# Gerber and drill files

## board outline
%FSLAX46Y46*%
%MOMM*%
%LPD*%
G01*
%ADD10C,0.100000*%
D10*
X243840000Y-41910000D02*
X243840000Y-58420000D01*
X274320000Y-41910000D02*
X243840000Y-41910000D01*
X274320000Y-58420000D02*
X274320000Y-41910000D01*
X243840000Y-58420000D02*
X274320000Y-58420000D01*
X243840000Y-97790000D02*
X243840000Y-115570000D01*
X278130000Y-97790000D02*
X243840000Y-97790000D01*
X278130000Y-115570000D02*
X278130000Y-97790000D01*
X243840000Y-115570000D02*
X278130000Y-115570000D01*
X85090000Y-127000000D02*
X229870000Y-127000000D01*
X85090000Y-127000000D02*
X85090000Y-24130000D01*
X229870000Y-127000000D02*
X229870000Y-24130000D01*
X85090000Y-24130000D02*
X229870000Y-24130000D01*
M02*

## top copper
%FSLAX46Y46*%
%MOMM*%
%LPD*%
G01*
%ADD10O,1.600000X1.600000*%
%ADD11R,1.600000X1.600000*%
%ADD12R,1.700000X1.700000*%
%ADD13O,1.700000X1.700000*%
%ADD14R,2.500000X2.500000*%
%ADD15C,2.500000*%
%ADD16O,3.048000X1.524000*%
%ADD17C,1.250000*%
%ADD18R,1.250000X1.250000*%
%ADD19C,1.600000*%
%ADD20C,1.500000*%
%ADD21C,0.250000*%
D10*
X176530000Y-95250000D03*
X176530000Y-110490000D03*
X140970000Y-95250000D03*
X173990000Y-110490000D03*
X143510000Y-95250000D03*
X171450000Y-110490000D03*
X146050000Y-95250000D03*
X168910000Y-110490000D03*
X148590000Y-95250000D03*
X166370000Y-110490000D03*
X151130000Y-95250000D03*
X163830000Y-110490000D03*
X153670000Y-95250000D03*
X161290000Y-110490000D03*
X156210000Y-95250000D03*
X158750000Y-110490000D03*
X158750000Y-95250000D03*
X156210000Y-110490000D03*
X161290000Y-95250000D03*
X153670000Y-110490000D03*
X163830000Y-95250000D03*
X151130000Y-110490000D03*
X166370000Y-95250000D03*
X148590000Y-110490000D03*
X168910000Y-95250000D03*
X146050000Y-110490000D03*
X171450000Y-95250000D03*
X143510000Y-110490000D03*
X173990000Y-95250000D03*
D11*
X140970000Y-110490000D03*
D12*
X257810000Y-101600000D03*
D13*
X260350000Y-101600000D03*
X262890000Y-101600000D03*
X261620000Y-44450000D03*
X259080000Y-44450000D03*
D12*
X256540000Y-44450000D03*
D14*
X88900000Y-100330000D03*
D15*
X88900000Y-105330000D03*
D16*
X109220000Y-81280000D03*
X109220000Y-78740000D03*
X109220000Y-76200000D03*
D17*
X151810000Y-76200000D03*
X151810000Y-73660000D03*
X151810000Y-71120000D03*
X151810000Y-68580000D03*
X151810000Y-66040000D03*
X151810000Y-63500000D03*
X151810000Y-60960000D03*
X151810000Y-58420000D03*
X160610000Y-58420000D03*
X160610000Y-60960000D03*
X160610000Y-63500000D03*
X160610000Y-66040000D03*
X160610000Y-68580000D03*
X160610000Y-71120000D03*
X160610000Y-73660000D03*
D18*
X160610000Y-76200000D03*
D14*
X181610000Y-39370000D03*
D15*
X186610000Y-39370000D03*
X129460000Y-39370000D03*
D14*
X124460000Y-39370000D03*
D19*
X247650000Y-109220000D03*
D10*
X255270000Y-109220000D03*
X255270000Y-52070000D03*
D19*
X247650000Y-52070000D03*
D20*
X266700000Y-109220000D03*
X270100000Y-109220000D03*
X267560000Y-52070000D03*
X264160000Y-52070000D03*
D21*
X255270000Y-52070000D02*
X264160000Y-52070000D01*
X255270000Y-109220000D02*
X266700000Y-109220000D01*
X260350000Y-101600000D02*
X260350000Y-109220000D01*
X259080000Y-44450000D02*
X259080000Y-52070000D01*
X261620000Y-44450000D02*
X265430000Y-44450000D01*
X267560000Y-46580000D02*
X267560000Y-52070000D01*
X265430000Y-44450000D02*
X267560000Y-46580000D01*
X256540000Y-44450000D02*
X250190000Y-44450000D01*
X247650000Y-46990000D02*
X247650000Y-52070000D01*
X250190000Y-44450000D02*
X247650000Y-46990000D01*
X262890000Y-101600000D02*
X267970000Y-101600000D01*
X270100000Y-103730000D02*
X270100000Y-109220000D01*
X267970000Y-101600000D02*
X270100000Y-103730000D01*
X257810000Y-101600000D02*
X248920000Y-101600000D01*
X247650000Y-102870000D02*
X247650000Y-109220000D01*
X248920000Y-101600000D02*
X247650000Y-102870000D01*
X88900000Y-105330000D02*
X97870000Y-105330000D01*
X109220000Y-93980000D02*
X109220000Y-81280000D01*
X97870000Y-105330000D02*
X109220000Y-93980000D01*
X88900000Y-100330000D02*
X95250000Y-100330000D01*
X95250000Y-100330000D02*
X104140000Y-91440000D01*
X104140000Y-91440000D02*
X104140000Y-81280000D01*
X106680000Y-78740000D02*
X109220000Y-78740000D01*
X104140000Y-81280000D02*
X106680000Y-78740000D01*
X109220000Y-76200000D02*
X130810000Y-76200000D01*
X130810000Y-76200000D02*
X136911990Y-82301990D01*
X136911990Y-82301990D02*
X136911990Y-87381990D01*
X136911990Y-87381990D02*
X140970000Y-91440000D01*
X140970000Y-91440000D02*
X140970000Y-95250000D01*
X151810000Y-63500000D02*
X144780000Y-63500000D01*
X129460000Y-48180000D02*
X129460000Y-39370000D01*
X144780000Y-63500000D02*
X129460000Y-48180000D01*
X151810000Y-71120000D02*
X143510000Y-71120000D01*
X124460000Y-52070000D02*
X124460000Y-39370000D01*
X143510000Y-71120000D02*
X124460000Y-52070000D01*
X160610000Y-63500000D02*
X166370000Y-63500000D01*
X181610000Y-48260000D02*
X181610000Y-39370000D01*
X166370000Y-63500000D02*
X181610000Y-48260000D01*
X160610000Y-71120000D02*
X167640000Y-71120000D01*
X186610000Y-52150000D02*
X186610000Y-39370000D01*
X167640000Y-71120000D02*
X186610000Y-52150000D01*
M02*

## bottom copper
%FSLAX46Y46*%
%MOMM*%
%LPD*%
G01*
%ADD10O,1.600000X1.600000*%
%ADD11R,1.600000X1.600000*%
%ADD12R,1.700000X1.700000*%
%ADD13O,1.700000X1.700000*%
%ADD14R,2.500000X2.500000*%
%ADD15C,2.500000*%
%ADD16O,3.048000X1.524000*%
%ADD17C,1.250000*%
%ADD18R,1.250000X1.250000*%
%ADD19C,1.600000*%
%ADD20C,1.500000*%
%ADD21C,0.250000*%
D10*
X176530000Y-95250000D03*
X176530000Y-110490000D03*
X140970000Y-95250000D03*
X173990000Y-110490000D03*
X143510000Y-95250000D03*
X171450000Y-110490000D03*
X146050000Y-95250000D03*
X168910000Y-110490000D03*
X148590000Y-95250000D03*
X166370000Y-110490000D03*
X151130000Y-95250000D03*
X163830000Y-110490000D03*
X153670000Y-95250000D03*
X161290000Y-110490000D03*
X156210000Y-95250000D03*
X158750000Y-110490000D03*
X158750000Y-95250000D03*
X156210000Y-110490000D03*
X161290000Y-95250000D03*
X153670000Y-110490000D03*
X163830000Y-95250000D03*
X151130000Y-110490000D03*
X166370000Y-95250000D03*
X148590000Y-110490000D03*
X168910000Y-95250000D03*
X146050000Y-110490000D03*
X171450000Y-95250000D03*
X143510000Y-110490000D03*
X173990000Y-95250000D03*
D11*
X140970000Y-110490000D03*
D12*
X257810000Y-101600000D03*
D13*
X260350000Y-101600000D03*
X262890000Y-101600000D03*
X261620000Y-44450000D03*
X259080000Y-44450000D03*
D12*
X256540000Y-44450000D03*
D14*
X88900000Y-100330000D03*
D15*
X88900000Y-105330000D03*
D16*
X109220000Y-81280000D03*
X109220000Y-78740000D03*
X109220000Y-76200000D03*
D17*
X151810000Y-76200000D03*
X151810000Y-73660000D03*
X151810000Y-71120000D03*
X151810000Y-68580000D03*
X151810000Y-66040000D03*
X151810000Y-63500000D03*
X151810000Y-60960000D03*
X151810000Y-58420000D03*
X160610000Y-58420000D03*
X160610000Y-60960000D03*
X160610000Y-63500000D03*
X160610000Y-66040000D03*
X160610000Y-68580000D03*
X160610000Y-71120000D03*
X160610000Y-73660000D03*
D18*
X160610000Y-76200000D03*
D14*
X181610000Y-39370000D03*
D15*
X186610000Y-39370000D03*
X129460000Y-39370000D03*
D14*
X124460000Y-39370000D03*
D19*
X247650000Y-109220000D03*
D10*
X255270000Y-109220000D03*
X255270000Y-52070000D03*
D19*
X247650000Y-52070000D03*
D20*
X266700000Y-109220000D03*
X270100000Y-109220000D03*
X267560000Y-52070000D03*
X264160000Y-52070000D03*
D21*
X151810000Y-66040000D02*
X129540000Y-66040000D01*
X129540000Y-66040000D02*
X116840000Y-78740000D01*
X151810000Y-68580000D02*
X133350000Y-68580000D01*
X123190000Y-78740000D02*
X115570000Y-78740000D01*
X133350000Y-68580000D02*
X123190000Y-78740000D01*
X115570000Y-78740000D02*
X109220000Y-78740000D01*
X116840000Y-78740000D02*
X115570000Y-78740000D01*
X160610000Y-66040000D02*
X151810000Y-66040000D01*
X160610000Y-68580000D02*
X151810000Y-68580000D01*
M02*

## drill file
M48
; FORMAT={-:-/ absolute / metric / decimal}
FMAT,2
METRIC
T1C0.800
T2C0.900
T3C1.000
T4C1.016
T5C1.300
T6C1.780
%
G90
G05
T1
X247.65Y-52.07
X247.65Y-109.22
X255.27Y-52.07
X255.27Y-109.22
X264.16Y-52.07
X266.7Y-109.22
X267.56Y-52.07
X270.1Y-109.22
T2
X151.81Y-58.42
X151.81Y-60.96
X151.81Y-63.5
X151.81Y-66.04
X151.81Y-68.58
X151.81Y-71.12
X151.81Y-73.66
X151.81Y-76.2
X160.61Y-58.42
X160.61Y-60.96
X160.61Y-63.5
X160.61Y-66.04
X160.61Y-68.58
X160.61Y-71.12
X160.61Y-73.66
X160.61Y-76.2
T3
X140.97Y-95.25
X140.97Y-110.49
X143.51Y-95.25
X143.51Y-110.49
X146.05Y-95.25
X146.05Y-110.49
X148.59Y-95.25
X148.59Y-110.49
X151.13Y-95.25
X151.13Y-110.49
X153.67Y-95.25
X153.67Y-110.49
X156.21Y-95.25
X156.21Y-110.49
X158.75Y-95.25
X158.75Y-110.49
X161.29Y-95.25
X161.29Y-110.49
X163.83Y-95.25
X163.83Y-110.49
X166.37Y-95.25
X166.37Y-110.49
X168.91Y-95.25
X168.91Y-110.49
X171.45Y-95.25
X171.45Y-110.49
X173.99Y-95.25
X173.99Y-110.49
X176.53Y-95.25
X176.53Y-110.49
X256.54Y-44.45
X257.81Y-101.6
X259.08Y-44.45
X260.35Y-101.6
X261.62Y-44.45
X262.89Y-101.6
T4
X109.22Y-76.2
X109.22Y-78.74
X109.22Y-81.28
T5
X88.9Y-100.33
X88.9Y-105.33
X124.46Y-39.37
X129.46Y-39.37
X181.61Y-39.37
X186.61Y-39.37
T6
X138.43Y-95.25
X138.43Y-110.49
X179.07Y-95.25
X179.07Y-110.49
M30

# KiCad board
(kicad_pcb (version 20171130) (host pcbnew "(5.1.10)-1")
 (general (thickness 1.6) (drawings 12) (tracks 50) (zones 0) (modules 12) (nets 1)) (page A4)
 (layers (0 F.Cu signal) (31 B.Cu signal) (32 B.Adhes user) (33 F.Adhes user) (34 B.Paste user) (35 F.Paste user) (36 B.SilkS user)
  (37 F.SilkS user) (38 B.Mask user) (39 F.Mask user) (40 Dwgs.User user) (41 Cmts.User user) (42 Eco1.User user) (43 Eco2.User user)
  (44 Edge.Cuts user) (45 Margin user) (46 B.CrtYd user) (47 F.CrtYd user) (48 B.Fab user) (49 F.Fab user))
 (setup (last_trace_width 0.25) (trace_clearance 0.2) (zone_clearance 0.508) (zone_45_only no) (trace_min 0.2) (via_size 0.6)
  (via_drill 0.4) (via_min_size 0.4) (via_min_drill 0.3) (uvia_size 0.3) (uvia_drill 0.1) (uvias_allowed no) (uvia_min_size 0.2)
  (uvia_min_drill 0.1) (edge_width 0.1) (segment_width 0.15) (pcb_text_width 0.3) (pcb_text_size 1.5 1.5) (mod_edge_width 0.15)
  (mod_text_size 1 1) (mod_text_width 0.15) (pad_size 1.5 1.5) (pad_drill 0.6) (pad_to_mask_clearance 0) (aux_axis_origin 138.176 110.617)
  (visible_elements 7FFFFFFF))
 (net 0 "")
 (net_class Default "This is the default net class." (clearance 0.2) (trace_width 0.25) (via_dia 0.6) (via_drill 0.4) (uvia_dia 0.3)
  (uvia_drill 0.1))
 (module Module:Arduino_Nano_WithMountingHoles (layer F.Cu) (at 140.97 110.49 90)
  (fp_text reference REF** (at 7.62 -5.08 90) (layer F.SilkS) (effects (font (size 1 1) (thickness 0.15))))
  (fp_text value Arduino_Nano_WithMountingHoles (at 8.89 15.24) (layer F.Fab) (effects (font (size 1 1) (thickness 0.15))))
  (pad "" np_thru_hole circle (at 0 38.1 90) (size 1.78 1.78) (drill 1.78) (layers *.Cu *.Mask))
  (pad "" np_thru_hole circle (at 15.24 38.1 90) (size 1.78 1.78) (drill 1.78) (layers *.Cu *.Mask))
  (pad "" np_thru_hole circle (at 15.24 -2.54 90) (size 1.78 1.78) (drill 1.78) (layers *.Cu *.Mask))
  (pad "" np_thru_hole circle (at 0 -2.54 90) (size 1.78 1.78) (drill 1.78) (layers *.Cu *.Mask))
  (pad 16 thru_hole oval (at 15.24 35.56 90) (size 1.6 1.6) (drill 1) (layers *.Cu *.Mask))
  (pad 15 thru_hole oval (at 0 35.56 90) (size 1.6 1.6) (drill 1) (layers *.Cu *.Mask))
  (pad 30 thru_hole oval (at 15.24 0 90) (size 1.6 1.6) (drill 1) (layers *.Cu *.Mask))
  (pad 14 thru_hole oval (at 0 33.02 90) (size 1.6 1.6) (drill 1) (layers *.Cu *.Mask))
  (pad 29 thru_hole oval (at 15.24 2.54 90) (size 1.6 1.6) (drill 1) (layers *.Cu *.Mask))
  (pad 13 thru_hole oval (at 0 30.48 90) (size 1.6 1.6) (drill 1) (layers *.Cu *.Mask))
  (pad 28 thru_hole oval (at 15.24 5.08 90) (size 1.6 1.6) (drill 1) (layers *.Cu *.Mask))
  (pad 12 thru_hole oval (at 0 27.94 90) (size 1.6 1.6) (drill 1) (layers *.Cu *.Mask))
  (pad 27 thru_hole oval (at 15.24 7.62 90) (size 1.6 1.6) (drill 1) (layers *.Cu *.Mask))
  (pad 11 thru_hole oval (at 0 25.4 90) (size 1.6 1.6) (drill 1) (layers *.Cu *.Mask))
  (pad 26 thru_hole oval (at 15.24 10.16 90) (size 1.6 1.6) (drill 1) (layers *.Cu *.Mask))
  (pad 10 thru_hole oval (at 0 22.86 90) (size 1.6 1.6) (drill 1) (layers *.Cu *.Mask))
  (pad 25 thru_hole oval (at 15.24 12.7 90) (size 1.6 1.6) (drill 1) (layers *.Cu *.Mask))
  (pad 9 thru_hole oval (at 0 20.32 90) (size 1.6 1.6) (drill 1) (layers *.Cu *.Mask))
  (pad 24 thru_hole oval (at 15.24 15.24 90) (size 1.6 1.6) (drill 1) (layers *.Cu *.Mask))
  (pad 8 thru_hole oval (at 0 17.78 90) (size 1.6 1.6) (drill 1) (layers *.Cu *.Mask))
  (pad 23 thru_hole oval (at 15.24 17.78 90) (size 1.6 1.6) (drill 1) (layers *.Cu *.Mask))
  (pad 7 thru_hole oval (at 0 15.24 90) (size 1.6 1.6) (drill 1) (layers *.Cu *.Mask))
  (pad 22 thru_hole oval (at 15.24 20.32 90) (size 1.6 1.6) (drill 1) (layers *.Cu *.Mask))
  (pad 6 thru_hole oval (at 0 12.7 90) (size 1.6 1.6) (drill 1) (layers *.Cu *.Mask))
  (pad 21 thru_hole oval (at 15.24 22.86 90) (size 1.6 1.6) (drill 1) (layers *.Cu *.Mask))
  (pad 5 thru_hole oval (at 0 10.16 90) (size 1.6 1.6) (drill 1) (layers *.Cu *.Mask))
  (pad 20 thru_hole oval (at 15.24 25.4 90) (size 1.6 1.6) (drill 1) (layers *.Cu *.Mask))
  (pad 4 thru_hole oval (at 0 7.62 90) (size 1.6 1.6) (drill 1) (layers *.Cu *.Mask))
  (pad 19 thru_hole oval (at 15.24 27.94 90) (size 1.6 1.6) (drill 1) (layers *.Cu *.Mask))
  (pad 3 thru_hole oval (at 0 5.08 90) (size 1.6 1.6) (drill 1) (layers *.Cu *.Mask))
  (pad 18 thru_hole oval (at 15.24 30.48 90) (size 1.6 1.6) (drill 1) (layers *.Cu *.Mask))
  (pad 2 thru_hole oval (at 0 2.54 90) (size 1.6 1.6) (drill 1) (layers *.Cu *.Mask))
  (pad 17 thru_hole oval (at 15.24 33.02 90) (size 1.6 1.6) (drill 1) (layers *.Cu *.Mask))
  (pad 1 thru_hole rect (at 0 0 90) (size 1.6 1.6) (drill 1) (layers *.Cu *.Mask)))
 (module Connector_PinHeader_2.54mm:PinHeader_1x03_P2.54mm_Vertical (layer F.Cu) (at 257.81 101.6 90)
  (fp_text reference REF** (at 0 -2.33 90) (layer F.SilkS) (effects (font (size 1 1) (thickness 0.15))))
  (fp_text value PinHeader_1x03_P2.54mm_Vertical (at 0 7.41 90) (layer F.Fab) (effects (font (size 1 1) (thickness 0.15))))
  (pad 1 thru_hole rect (at 0 0 90) (size 1.7 1.7) (drill 1) (layers *.Cu *.Mask))
  (pad 2 thru_hole oval (at 0 2.54 90) (size 1.7 1.7) (drill 1) (layers *.Cu *.Mask))
  (pad 3 thru_hole oval (at 0 5.08 90) (size 1.7 1.7) (drill 1) (layers *.Cu *.Mask)))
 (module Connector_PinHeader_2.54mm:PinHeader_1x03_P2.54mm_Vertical (layer F.Cu) (at 256.54 44.45 90)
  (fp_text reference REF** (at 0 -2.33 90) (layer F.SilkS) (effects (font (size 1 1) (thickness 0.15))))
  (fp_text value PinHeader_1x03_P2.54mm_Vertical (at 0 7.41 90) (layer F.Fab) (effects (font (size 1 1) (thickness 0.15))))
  (pad 3 thru_hole oval (at 0 5.08 90) (size 1.7 1.7) (drill 1) (layers *.Cu *.Mask))
  (pad 2 thru_hole oval (at 0 2.54 90) (size 1.7 1.7) (drill 1) (layers *.Cu *.Mask))
  (pad 1 thru_hole rect (at 0 0 90) (size 1.7 1.7) (drill 1) (layers *.Cu *.Mask)))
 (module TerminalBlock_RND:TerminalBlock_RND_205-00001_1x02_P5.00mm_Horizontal (layer F.Cu) (at 88.9 100.33 270)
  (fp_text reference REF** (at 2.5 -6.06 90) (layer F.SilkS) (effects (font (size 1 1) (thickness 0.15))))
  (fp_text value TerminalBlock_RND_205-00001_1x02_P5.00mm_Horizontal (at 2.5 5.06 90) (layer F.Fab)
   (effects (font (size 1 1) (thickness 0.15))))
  (pad 1 thru_hole rect (at 0 0 270) (size 2.5 2.5) (drill 1.3) (layers *.Cu *.Mask))
  (pad 2 thru_hole circle (at 5 0 270) (size 2.5 2.5) (drill 1.3) (layers *.Cu *.Mask)))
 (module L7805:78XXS (layer F.Cu) (at 111.76 78.74 270)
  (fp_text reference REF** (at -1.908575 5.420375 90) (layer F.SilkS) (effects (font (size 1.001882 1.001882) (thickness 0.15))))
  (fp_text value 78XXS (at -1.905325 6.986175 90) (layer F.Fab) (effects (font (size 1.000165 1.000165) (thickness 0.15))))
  (pad OUT thru_hole oval (at 2.54 2.54 270) (size 1.524 3.048) (drill 1.016) (layers *.Cu *.Mask))
  (pad GND thru_hole oval (at 0 2.54 270) (size 1.524 3.048) (drill 1.016) (layers *.Cu *.Mask))
  (pad IN thru_hole oval (at -2.54 2.54 270) (size 1.524 3.048) (drill 1.016) (layers *.Cu *.Mask)))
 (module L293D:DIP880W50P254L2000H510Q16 (layer F.Cu) (at 156.21 67.31 180)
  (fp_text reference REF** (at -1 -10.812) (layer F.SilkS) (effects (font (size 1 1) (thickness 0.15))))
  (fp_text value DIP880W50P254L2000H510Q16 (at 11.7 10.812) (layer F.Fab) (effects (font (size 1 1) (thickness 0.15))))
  (pad 16 thru_hole circle (at 4.4 -8.89 180) (size 1.25 1.25) (drill 0.9) (layers *.Cu *.Mask))
  (pad 15 thru_hole circle (at 4.4 -6.35 180) (size 1.25 1.25) (drill 0.9) (layers *.Cu *.Mask))
  (pad 14 thru_hole circle (at 4.4 -3.81 180) (size 1.25 1.25) (drill 0.9) (layers *.Cu *.Mask))
  (pad 13 thru_hole circle (at 4.4 -1.27 180) (size 1.25 1.25) (drill 0.9) (layers *.Cu *.Mask))
  (pad 12 thru_hole circle (at 4.4 1.27 180) (size 1.25 1.25) (drill 0.9) (layers *.Cu *.Mask))
  (pad 11 thru_hole circle (at 4.4 3.81 180) (size 1.25 1.25) (drill 0.9) (layers *.Cu *.Mask))
  (pad 10 thru_hole circle (at 4.4 6.35 180) (size 1.25 1.25) (drill 0.9) (layers *.Cu *.Mask))
  (pad 9 thru_hole circle (at 4.4 8.89 180) (size 1.25 1.25) (drill 0.9) (layers *.Cu *.Mask))
  (pad 8 thru_hole circle (at -4.4 8.89 180) (size 1.25 1.25) (drill 0.9) (layers *.Cu *.Mask))
  (pad 7 thru_hole circle (at -4.4 6.35 180) (size 1.25 1.25) (drill 0.9) (layers *.Cu *.Mask))
  (pad 6 thru_hole circle (at -4.4 3.81 180) (size 1.25 1.25) (drill 0.9) (layers *.Cu *.Mask))
  (pad 5 thru_hole circle (at -4.4 1.27 180) (size 1.25 1.25) (drill 0.9) (layers *.Cu *.Mask))
  (pad 4 thru_hole circle (at -4.4 -1.27 180) (size 1.25 1.25) (drill 0.9) (layers *.Cu *.Mask))
  (pad 3 thru_hole circle (at -4.4 -3.81 180) (size 1.25 1.25) (drill 0.9) (layers *.Cu *.Mask))
  (pad 2 thru_hole circle (at -4.4 -6.35 180) (size 1.25 1.25) (drill 0.9) (layers *.Cu *.Mask))
  (pad 1 thru_hole rect (at -4.4 -8.89 180) (size 1.25 1.25) (drill 0.9) (layers *.Cu *.Mask)))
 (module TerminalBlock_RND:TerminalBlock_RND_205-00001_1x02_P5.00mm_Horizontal (layer F.Cu) (at 181.61 39.37)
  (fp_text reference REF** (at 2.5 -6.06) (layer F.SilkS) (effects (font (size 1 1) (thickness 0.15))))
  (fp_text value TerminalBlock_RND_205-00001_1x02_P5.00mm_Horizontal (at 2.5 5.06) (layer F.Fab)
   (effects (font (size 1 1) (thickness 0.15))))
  (pad 1 thru_hole rect (at 0 0) (size 2.5 2.5) (drill 1.3) (layers *.Cu *.Mask))
  (pad 2 thru_hole circle (at 5 0) (size 2.5 2.5) (drill 1.3) (layers *.Cu *.Mask)))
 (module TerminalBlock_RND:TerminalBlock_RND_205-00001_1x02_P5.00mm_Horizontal (layer F.Cu) (at 124.46 39.37)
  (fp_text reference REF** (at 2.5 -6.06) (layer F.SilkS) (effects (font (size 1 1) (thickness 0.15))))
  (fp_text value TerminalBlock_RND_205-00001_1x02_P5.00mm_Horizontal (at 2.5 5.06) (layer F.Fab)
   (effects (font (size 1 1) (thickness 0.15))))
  (pad 2 thru_hole circle (at 5 0) (size 2.5 2.5) (drill 1.3) (layers *.Cu *.Mask))
  (pad 1 thru_hole rect (at 0 0) (size 2.5 2.5) (drill 1.3) (layers *.Cu *.Mask)))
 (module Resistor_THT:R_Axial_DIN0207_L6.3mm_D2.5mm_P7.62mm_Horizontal (layer F.Cu) (at 247.65 109.22)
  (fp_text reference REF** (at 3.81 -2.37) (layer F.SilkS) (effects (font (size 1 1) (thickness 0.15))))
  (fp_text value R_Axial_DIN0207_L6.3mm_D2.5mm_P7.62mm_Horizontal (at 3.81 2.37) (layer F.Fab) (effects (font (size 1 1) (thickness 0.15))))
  (pad 1 thru_hole circle (at 0 0) (size 1.6 1.6) (drill 0.8) (layers *.Cu *.Mask))
  (pad 2 thru_hole oval (at 7.62 0) (size 1.6 1.6) (drill 0.8) (layers *.Cu *.Mask)))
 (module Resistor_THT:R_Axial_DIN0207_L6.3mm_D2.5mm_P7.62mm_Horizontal (layer F.Cu) (at 247.65 52.07)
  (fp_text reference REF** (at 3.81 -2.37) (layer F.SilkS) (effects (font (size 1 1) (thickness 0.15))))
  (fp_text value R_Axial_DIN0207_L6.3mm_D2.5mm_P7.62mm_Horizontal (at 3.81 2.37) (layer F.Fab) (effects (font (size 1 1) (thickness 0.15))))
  (pad 2 thru_hole oval (at 7.62 0) (size 1.6 1.6) (drill 0.8) (layers *.Cu *.Mask))
  (pad 1 thru_hole circle (at 0 0) (size 1.6 1.6) (drill 0.8) (layers *.Cu *.Mask)))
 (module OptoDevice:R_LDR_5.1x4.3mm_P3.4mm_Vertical (layer F.Cu) (at 266.7 109.22)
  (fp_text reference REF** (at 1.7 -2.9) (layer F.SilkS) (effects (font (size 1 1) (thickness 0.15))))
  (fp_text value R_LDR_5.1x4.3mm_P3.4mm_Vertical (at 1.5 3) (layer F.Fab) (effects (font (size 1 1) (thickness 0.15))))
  (pad 1 thru_hole circle (at 0 0) (size 1.5 1.5) (drill 0.8) (layers *.Cu *.Mask))
  (pad 2 thru_hole circle (at 3.4 0) (size 1.5 1.5) (drill 0.8) (layers *.Cu *.Mask)))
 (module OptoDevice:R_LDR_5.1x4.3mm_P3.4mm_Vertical (layer F.Cu) (at 264.16 52.07)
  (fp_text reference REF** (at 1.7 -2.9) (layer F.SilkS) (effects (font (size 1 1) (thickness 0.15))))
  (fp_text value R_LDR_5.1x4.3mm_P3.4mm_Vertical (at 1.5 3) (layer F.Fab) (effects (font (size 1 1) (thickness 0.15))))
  (pad 2 thru_hole circle (at 3.4 0) (size 1.5 1.5) (drill 0.8) (layers *.Cu *.Mask))
  (pad 1 thru_hole circle (at 0 0) (size 1.5 1.5) (drill 0.8) (layers *.Cu *.Mask)))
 (gr_line (start 243.84 41.91) (end 243.84 58.42) (layer Edge.Cuts) (width 0.1))
 (gr_line (start 274.32 41.91) (end 243.84 41.91) (layer Edge.Cuts) (width 0.1))
 (gr_line (start 274.32 58.42) (end 274.32 41.91) (layer Edge.Cuts) (width 0.1))
 (gr_line (start 243.84 58.42) (end 274.32 58.42) (layer Edge.Cuts) (width 0.1))
 (gr_line (start 243.84 97.79) (end 243.84 115.57) (layer Edge.Cuts) (width 0.1))
 (gr_line (start 278.13 97.79) (end 243.84 97.79) (layer Edge.Cuts) (width 0.1))
 (gr_line (start 278.13 115.57) (end 278.13 97.79) (layer Edge.Cuts) (width 0.1))
 (gr_line (start 243.84 115.57) (end 278.13 115.57) (layer Edge.Cuts) (width 0.1))
 (gr_line (start 85.09 127) (end 229.87 127) (layer Edge.Cuts) (width 0.1))
 (gr_line (start 85.09 127) (end 85.09 24.13) (layer Edge.Cuts) (width 0.1))
 (gr_line (start 229.87 127) (end 229.87 24.13) (layer Edge.Cuts) (width 0.1))
 (gr_line (start 85.09 24.13) (end 229.87 24.13) (layer Edge.Cuts) (width 0.1))
 (segment (start 255.27 52.07) (end 264.16 52.07) (width 0.25) (layer F.Cu) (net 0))
 (segment (start 255.27 109.22) (end 266.7 109.22) (width 0.25) (layer F.Cu) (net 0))
 (segment (start 260.35 101.6) (end 260.35 109.22) (width 0.25) (layer F.Cu) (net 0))
 (segment (start 259.08 44.45) (end 259.08 52.07) (width 0.25) (layer F.Cu) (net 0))
 (segment (start 261.62 44.45) (end 265.43 44.45) (width 0.25) (layer F.Cu) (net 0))
 (segment (start 267.56 46.58) (end 267.56 52.07) (width 0.25) (layer F.Cu) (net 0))
 (segment (start 265.43 44.45) (end 267.56 46.58) (width 0.25) (layer F.Cu) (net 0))
 (segment (start 256.54 44.45) (end 250.19 44.45) (width 0.25) (layer F.Cu) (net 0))
 (segment (start 247.65 46.99) (end 247.65 52.07) (width 0.25) (layer F.Cu) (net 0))
 (segment (start 250.19 44.45) (end 247.65 46.99) (width 0.25) (layer F.Cu) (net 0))
 (segment (start 262.89 101.6) (end 267.97 101.6) (width 0.25) (layer F.Cu) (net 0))
 (segment (start 270.1 103.73) (end 270.1 109.22) (width 0.25) (layer F.Cu) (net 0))
 (segment (start 267.97 101.6) (end 270.1 103.73) (width 0.25) (layer F.Cu) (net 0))
 (segment (start 257.81 101.6) (end 248.92 101.6) (width 0.25) (layer F.Cu) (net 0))
 (segment (start 247.65 102.87) (end 247.65 109.22) (width 0.25) (layer F.Cu) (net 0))
 (segment (start 248.92 101.6) (end 247.65 102.87) (width 0.25) (layer F.Cu) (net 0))
 (segment (start 88.9 105.33) (end 97.87 105.33) (width 0.25) (layer F.Cu) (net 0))
 (segment (start 109.22 93.98) (end 109.22 81.28) (width 0.25) (layer F.Cu) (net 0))
 (segment (start 97.87 105.33) (end 109.22 93.98) (width 0.25) (layer F.Cu) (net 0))
 (segment (start 88.9 100.33) (end 95.25 100.33) (width 0.25) (layer F.Cu) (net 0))
 (segment (start 95.25 100.33) (end 104.14 91.44) (width 0.25) (layer F.Cu) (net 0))
 (segment (start 104.14 91.44) (end 104.14 81.28) (width 0.25) (layer F.Cu) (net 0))
 (segment (start 106.68 78.74) (end 109.22 78.74) (width 0.25) (layer F.Cu) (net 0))
 (segment (start 104.14 81.28) (end 106.68 78.74) (width 0.25) (layer F.Cu) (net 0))
 (segment (start 109.22 76.2) (end 130.81 76.2) (width 0.25) (layer F.Cu) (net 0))
 (segment (start 130.81 76.2) (end 136.91199 82.30199) (width 0.25) (layer F.Cu) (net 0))
 (segment (start 136.91199 82.30199) (end 136.91199 87.38199) (width 0.25) (layer F.Cu) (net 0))
 (segment (start 136.91199 87.38199) (end 140.97 91.44) (width 0.25) (layer F.Cu) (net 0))
 (segment (start 140.97 91.44) (end 140.97 95.25) (width 0.25) (layer F.Cu) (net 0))
 (segment (start 151.81 63.5) (end 144.78 63.5) (width 0.25) (layer F.Cu) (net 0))
 (segment (start 129.46 48.18) (end 129.46 39.37) (width 0.25) (layer F.Cu) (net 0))
 (segment (start 144.78 63.5) (end 129.46 48.18) (width 0.25) (layer F.Cu) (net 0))
 (segment (start 151.81 71.12) (end 143.51 71.12) (width 0.25) (layer F.Cu) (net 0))
 (segment (start 124.46 52.07) (end 124.46 39.37) (width 0.25) (layer F.Cu) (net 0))
 (segment (start 143.51 71.12) (end 124.46 52.07) (width 0.25) (layer F.Cu) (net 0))
 (segment (start 160.61 63.5) (end 166.37 63.5) (width 0.25) (layer F.Cu) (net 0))
 (segment (start 181.61 48.26) (end 181.61 39.37) (width 0.25) (layer F.Cu) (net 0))
 (segment (start 166.37 63.5) (end 181.61 48.26) (width 0.25) (layer F.Cu) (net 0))
 (segment (start 160.61 71.12) (end 167.64 71.12) (width 0.25) (layer F.Cu) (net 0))
 (segment (start 186.61 52.15) (end 186.61 39.37) (width 0.25) (layer F.Cu) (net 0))
 (segment (start 167.64 71.12) (end 186.61 52.15) (width 0.25) (layer F.Cu) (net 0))
 (segment (start 151.81 66.04) (end 129.54 66.04) (width 0.25) (layer B.Cu) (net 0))
 (segment (start 129.54 66.04) (end 116.84 78.74) (width 0.25) (layer B.Cu) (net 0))
 (segment (start 151.81 68.58) (end 133.35 68.58) (width 0.25) (layer B.Cu) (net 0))
 (segment (start 123.19 78.74) (end 115.57 78.74) (width 0.25) (layer B.Cu) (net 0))
 (segment (start 133.35 68.58) (end 123.19 78.74) (width 0.25) (layer B.Cu) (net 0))
 (segment (start 115.57 78.74) (end 109.22 78.74) (width 0.25) (layer B.Cu) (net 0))
 (segment (start 116.84 78.74) (end 115.57 78.74) (width 0.25) (layer B.Cu) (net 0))
 (segment (start 160.61 66.04) (end 151.81 66.04) (width 0.25) (layer B.Cu) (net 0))
 (segment (start 160.61 68.58) (end 151.81 68.58) (width 0.25) (layer B.Cu) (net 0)))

